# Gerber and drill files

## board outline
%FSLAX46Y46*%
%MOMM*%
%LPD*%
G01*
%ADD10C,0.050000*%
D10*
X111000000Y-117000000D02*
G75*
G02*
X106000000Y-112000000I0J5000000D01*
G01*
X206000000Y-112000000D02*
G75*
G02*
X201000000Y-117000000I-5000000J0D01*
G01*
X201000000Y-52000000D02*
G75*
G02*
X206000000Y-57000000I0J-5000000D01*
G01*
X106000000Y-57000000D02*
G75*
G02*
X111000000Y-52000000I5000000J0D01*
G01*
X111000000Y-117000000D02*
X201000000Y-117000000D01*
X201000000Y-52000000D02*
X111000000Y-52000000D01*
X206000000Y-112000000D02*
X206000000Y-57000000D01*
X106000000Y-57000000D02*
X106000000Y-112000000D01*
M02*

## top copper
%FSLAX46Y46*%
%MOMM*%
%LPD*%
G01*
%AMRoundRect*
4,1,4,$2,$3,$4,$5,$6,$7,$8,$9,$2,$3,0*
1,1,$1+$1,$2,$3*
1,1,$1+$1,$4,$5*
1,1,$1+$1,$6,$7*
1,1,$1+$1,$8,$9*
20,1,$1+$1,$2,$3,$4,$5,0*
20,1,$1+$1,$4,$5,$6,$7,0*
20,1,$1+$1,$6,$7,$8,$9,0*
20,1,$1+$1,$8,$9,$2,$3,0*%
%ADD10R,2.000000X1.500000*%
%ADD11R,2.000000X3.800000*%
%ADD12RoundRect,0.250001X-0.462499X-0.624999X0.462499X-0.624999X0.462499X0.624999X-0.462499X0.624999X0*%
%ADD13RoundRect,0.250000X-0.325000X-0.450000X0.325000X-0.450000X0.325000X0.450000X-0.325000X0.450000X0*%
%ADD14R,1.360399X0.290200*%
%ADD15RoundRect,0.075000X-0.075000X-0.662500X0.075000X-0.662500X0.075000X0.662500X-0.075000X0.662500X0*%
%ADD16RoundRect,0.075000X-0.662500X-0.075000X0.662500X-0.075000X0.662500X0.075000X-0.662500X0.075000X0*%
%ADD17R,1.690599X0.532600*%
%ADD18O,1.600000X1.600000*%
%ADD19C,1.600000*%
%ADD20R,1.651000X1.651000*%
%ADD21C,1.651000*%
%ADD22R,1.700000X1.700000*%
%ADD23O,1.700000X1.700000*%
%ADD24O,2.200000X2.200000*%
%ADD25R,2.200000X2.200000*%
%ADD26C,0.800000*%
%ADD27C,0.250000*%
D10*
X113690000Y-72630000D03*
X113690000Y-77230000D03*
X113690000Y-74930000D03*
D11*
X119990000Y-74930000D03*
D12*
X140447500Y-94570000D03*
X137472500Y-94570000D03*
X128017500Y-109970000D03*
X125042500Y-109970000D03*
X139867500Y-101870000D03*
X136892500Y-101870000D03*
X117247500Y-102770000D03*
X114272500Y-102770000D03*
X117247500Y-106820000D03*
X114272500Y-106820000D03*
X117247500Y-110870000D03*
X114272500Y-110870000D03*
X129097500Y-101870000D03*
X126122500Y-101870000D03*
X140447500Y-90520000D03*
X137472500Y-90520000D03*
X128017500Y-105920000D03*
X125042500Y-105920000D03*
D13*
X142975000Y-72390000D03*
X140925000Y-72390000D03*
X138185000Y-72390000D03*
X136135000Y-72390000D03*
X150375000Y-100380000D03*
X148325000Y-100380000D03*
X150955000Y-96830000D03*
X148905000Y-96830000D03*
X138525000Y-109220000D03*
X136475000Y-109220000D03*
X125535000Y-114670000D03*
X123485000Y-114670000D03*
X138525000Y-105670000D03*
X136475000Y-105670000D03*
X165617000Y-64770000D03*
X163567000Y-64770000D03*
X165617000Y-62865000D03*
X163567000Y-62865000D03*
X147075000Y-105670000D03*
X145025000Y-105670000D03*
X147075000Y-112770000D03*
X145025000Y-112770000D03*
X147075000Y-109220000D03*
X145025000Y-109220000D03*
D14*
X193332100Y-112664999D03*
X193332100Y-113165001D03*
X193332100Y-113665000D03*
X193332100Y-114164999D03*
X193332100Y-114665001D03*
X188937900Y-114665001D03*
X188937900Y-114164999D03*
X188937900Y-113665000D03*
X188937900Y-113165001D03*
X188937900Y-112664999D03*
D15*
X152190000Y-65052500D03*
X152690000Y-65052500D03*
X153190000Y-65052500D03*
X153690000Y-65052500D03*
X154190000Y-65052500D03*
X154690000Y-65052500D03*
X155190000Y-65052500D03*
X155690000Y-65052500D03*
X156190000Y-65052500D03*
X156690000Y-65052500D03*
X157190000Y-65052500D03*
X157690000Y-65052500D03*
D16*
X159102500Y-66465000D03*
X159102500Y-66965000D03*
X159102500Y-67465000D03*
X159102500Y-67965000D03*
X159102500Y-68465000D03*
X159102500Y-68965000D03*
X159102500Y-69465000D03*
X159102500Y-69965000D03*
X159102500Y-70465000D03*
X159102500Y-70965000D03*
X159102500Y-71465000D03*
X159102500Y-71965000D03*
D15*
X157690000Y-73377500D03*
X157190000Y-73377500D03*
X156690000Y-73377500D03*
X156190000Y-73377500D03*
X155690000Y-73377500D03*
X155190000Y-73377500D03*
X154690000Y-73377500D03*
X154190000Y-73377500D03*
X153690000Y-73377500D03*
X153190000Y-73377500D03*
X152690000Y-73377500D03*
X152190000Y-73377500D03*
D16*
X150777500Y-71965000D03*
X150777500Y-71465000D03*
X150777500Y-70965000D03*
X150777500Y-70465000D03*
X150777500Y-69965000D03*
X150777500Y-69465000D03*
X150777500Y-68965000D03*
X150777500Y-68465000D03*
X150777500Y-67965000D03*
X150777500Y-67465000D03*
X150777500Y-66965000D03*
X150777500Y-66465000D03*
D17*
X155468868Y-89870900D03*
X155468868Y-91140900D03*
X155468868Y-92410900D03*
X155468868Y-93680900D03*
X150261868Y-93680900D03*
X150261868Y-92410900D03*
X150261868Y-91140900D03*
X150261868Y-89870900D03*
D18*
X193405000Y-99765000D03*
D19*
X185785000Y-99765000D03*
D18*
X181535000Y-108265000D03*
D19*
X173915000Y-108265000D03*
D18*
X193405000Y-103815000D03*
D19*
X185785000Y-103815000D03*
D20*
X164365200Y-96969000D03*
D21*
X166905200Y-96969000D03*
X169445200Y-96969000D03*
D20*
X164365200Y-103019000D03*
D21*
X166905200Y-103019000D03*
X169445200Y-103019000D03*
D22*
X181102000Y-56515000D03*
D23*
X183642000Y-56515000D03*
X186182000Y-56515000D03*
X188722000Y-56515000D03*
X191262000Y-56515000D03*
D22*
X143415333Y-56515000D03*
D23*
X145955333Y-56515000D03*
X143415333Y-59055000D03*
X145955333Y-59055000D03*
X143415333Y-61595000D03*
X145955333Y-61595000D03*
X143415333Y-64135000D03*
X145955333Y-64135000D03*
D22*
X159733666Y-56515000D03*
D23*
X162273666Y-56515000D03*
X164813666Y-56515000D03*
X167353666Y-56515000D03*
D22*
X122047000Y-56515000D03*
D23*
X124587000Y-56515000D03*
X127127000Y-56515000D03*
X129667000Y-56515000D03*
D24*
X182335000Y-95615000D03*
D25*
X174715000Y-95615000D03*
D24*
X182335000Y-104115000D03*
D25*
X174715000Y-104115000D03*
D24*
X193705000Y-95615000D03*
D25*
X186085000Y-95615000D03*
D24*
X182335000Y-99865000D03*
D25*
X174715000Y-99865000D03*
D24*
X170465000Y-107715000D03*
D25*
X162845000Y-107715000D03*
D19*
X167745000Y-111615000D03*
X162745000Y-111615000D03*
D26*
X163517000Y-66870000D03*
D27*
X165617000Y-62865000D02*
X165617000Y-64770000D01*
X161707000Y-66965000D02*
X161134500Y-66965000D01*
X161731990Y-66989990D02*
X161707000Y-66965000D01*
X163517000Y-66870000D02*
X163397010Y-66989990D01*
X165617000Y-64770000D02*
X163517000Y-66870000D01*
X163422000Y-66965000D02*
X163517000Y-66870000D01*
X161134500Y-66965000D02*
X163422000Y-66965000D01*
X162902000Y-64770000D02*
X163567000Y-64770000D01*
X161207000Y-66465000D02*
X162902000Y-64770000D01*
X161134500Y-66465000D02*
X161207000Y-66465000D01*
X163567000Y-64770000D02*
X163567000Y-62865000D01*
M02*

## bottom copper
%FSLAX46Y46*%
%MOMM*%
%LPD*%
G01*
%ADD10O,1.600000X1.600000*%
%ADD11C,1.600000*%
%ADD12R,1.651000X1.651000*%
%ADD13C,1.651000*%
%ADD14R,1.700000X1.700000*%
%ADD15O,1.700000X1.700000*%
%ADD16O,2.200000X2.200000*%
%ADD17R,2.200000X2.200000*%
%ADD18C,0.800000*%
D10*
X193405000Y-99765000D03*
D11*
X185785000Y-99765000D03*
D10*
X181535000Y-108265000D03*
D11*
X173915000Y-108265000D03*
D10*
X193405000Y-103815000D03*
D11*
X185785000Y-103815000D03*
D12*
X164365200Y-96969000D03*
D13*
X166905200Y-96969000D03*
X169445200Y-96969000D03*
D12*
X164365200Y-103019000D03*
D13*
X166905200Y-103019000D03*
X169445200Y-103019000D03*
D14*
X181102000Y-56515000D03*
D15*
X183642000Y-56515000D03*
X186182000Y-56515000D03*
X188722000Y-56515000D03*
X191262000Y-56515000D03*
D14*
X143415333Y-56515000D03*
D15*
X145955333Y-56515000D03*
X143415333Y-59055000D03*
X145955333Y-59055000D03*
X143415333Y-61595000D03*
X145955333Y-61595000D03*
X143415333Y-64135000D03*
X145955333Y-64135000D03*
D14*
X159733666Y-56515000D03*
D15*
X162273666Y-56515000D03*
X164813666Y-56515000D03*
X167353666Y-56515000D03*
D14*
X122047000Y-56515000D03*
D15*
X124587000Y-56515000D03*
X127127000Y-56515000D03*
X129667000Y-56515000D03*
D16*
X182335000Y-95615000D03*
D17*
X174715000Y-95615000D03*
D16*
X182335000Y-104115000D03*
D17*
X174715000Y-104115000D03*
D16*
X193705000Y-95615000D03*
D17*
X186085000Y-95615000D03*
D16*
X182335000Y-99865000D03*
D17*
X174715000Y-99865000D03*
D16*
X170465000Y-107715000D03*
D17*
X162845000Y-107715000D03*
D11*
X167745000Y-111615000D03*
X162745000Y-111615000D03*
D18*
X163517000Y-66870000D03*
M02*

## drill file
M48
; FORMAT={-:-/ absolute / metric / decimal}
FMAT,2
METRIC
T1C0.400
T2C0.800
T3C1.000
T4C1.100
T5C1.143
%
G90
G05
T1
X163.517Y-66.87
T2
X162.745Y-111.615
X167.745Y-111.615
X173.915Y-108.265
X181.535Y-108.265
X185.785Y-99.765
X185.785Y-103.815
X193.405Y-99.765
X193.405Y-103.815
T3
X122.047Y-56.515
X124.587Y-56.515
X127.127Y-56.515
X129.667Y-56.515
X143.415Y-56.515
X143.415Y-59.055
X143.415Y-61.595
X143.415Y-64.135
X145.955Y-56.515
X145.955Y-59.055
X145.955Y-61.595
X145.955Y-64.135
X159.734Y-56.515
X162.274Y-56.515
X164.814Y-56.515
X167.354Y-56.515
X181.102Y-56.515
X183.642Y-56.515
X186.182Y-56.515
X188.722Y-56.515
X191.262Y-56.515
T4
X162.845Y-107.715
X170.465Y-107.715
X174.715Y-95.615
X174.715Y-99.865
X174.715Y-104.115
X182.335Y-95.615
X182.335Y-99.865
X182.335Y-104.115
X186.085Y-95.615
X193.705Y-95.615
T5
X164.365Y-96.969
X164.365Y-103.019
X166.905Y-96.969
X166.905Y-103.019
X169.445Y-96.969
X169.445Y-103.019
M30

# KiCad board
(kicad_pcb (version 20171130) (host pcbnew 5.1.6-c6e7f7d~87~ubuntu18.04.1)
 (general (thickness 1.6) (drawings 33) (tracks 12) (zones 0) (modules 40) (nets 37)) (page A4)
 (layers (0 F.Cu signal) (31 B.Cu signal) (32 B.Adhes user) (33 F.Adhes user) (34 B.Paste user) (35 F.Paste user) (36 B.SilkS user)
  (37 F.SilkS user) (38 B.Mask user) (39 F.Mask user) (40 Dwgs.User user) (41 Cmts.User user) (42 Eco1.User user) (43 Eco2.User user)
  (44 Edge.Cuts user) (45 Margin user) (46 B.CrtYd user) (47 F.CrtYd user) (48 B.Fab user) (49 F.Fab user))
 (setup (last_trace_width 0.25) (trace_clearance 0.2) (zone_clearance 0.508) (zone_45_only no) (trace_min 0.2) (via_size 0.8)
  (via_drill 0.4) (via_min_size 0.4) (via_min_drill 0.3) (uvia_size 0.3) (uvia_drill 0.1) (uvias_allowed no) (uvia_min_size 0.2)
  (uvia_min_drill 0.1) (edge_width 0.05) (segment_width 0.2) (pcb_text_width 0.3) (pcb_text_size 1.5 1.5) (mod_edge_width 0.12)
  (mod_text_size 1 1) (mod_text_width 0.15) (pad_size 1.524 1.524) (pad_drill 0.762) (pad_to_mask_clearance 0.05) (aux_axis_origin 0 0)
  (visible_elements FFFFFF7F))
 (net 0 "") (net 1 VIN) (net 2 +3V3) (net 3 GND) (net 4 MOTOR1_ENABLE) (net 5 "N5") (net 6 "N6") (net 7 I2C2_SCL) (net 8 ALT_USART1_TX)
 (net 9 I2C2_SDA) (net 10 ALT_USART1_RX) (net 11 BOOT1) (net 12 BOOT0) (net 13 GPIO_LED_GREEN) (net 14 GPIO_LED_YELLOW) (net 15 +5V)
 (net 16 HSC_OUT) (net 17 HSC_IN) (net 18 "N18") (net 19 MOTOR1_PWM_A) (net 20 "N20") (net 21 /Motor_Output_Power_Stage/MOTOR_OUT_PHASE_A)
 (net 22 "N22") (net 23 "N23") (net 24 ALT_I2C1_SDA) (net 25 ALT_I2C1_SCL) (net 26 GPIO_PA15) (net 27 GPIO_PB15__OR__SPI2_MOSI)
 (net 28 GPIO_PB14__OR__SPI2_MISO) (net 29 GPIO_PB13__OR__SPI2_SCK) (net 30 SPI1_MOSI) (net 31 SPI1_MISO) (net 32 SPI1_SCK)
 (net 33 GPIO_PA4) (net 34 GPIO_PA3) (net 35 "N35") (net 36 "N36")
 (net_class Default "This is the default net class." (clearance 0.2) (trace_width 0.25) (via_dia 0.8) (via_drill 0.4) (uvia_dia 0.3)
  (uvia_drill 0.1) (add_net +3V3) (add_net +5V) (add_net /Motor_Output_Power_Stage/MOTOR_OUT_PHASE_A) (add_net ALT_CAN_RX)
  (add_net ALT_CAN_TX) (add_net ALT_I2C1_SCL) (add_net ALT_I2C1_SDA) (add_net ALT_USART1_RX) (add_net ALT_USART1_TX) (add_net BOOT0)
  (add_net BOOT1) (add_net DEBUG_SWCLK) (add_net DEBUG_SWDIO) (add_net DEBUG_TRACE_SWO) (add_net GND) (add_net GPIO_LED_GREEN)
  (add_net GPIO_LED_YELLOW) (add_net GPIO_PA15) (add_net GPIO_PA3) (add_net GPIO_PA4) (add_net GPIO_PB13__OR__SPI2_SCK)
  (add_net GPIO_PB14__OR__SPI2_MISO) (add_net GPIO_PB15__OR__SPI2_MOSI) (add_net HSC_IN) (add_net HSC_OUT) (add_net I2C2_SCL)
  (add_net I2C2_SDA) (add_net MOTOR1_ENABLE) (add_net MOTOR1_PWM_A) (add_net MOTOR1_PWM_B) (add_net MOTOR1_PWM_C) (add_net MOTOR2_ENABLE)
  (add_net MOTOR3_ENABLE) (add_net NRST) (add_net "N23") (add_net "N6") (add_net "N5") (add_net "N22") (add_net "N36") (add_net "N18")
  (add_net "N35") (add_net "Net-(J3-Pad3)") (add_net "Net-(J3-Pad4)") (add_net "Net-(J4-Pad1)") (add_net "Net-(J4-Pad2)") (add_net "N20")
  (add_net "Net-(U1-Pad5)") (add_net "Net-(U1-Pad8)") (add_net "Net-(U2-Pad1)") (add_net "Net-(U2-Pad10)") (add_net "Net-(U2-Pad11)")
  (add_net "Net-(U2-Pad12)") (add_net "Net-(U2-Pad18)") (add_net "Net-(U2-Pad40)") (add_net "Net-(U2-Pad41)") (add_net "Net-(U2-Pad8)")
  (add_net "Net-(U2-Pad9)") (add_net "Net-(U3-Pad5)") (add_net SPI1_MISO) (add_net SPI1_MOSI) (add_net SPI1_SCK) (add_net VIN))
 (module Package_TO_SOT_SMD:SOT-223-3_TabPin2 (layer F.Cu) (at 116.84 74.93)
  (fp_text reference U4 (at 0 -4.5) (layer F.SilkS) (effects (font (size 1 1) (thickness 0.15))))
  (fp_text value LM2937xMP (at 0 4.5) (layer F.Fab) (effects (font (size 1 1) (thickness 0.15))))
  (pad 1 smd rect (at -3.15 -2.3) (size 2 1.5) (layers F.Cu F.Paste F.Mask) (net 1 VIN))
  (pad 3 smd rect (at -3.15 2.3) (size 2 1.5) (layers F.Cu F.Paste F.Mask) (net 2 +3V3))
  (pad 2 smd rect (at -3.15 0) (size 2 1.5) (layers F.Cu F.Paste F.Mask) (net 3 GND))
  (pad 2 smd rect (at 3.15 0) (size 2 3.8) (layers F.Cu F.Paste F.Mask) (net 3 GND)))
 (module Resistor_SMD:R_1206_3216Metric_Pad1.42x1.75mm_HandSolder (layer F.Cu) (at 138.96 94.57)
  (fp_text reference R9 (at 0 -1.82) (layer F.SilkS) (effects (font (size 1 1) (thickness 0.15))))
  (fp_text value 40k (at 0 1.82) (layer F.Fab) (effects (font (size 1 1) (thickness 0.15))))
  (pad 2 smd roundrect (at 1.4875 0) (size 1.425 1.75) (layers F.Cu F.Paste F.Mask) (roundrect_rratio 0.175439) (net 3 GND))
  (pad 1 smd roundrect (at -1.4875 0) (size 1.425 1.75) (layers F.Cu F.Paste F.Mask) (roundrect_rratio 0.175439) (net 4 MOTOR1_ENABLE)))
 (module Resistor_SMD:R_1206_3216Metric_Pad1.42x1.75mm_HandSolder (layer F.Cu) (at 126.53 109.97)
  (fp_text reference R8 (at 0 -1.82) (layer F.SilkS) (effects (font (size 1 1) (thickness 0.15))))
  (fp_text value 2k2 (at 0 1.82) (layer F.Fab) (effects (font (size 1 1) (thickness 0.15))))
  (pad 2 smd roundrect (at 1.4875 0) (size 1.425 1.75) (layers F.Cu F.Paste F.Mask) (roundrect_rratio 0.175439) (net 3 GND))
  (pad 1 smd roundrect (at -1.4875 0) (size 1.425 1.75) (layers F.Cu F.Paste F.Mask) (roundrect_rratio 0.175439) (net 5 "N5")))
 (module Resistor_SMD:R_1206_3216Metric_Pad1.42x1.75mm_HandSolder (layer F.Cu) (at 138.38 101.87)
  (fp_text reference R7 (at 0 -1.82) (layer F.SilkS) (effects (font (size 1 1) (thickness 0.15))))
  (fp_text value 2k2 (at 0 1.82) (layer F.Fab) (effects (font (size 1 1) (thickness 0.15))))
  (pad 2 smd roundrect (at 1.4875 0) (size 1.425 1.75) (layers F.Cu F.Paste F.Mask) (roundrect_rratio 0.175439) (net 3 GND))
  (pad 1 smd roundrect (at -1.4875 0) (size 1.425 1.75) (layers F.Cu F.Paste F.Mask) (roundrect_rratio 0.175439) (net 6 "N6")))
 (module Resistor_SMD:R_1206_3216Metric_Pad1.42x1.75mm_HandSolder (layer F.Cu) (at 115.76 102.77)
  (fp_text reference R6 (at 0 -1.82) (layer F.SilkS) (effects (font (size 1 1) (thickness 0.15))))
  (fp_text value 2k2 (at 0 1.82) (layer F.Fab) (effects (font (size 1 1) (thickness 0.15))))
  (pad 2 smd roundrect (at 1.4875 0) (size 1.425 1.75) (layers F.Cu F.Paste F.Mask) (roundrect_rratio 0.175439) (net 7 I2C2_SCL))
  (pad 1 smd roundrect (at -1.4875 0) (size 1.425 1.75) (layers F.Cu F.Paste F.Mask) (roundrect_rratio 0.175439) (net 2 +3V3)))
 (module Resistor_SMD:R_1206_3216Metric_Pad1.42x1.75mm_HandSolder (layer F.Cu) (at 115.76 106.82)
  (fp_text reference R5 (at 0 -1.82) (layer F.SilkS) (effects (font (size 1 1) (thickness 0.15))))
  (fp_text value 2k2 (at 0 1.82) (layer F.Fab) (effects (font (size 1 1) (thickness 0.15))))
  (pad 2 smd roundrect (at 1.4875 0) (size 1.425 1.75) (layers F.Cu F.Paste F.Mask) (roundrect_rratio 0.175439) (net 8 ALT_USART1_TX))
  (pad 1 smd roundrect (at -1.4875 0) (size 1.425 1.75) (layers F.Cu F.Paste F.Mask) (roundrect_rratio 0.175439) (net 2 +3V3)))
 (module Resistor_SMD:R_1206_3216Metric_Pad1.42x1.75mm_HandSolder (layer F.Cu) (at 115.76 110.87)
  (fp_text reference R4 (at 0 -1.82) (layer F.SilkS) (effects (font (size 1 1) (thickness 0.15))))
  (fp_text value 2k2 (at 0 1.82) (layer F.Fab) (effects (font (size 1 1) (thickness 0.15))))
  (pad 2 smd roundrect (at 1.4875 0) (size 1.425 1.75) (layers F.Cu F.Paste F.Mask) (roundrect_rratio 0.175439) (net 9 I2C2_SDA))
  (pad 1 smd roundrect (at -1.4875 0) (size 1.425 1.75) (layers F.Cu F.Paste F.Mask) (roundrect_rratio 0.175439) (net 2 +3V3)))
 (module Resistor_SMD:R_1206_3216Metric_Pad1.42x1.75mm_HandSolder (layer F.Cu) (at 127.61 101.87)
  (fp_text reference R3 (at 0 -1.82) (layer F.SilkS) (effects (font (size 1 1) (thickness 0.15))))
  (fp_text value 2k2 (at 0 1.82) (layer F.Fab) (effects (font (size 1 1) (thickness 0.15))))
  (pad 2 smd roundrect (at 1.4875 0) (size 1.425 1.75) (layers F.Cu F.Paste F.Mask) (roundrect_rratio 0.175439) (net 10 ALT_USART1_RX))
  (pad 1 smd roundrect (at -1.4875 0) (size 1.425 1.75) (layers F.Cu F.Paste F.Mask) (roundrect_rratio 0.175439) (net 2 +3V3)))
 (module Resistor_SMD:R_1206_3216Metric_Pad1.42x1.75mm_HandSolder (layer F.Cu) (at 138.96 90.52)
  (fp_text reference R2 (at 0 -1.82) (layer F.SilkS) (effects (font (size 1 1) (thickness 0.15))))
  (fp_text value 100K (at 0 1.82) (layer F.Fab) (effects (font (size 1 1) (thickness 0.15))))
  (pad 2 smd roundrect (at 1.4875 0) (size 1.425 1.75) (layers F.Cu F.Paste F.Mask) (roundrect_rratio 0.175439))
  (pad 1 smd roundrect (at -1.4875 0) (size 1.425 1.75) (layers F.Cu F.Paste F.Mask) (roundrect_rratio 0.175439) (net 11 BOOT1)))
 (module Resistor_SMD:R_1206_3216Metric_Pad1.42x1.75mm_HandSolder (layer F.Cu) (at 126.53 105.92)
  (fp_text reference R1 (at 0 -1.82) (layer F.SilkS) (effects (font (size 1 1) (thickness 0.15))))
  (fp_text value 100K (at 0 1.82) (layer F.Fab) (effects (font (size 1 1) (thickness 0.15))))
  (pad 2 smd roundrect (at 1.4875 0) (size 1.425 1.75) (layers F.Cu F.Paste F.Mask) (roundrect_rratio 0.175439) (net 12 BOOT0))
  (pad 1 smd roundrect (at -1.4875 0) (size 1.425 1.75) (layers F.Cu F.Paste F.Mask) (roundrect_rratio 0.175439)))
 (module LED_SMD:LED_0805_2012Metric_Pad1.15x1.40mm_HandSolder (layer F.Cu) (at 141.95 72.39)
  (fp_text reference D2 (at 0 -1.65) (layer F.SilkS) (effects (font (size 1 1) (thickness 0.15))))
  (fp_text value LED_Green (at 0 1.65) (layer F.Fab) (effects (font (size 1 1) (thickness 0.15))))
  (pad 2 smd roundrect (at 1.025 0) (size 1.15 1.4) (layers F.Cu F.Paste F.Mask) (roundrect_rratio 0.217391) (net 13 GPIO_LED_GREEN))
  (pad 1 smd roundrect (at -1.025 0) (size 1.15 1.4) (layers F.Cu F.Paste F.Mask) (roundrect_rratio 0.217391) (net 5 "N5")))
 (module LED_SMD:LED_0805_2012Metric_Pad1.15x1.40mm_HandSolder (layer F.Cu) (at 137.16 72.39)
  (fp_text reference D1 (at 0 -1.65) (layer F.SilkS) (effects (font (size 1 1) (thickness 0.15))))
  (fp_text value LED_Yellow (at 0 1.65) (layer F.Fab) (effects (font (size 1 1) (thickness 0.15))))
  (pad 2 smd roundrect (at 1.025 0) (size 1.15 1.4) (layers F.Cu F.Paste F.Mask) (roundrect_rratio 0.217391) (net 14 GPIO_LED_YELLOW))
  (pad 1 smd roundrect (at -1.025 0) (size 1.15 1.4) (layers F.Cu F.Paste F.Mask) (roundrect_rratio 0.217391) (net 6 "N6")))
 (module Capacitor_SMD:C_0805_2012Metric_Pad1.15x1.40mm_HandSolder (layer F.Cu) (at 149.35 100.38)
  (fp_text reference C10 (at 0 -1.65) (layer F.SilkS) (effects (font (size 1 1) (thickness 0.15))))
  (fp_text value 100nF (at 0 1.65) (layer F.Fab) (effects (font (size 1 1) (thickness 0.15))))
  (pad 2 smd roundrect (at 1.025 0) (size 1.15 1.4) (layers F.Cu F.Paste F.Mask) (roundrect_rratio 0.217391) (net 3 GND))
  (pad 1 smd roundrect (at -1.025 0) (size 1.15 1.4) (layers F.Cu F.Paste F.Mask) (roundrect_rratio 0.217391) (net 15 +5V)))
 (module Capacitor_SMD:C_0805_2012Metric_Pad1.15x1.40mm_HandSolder (layer F.Cu) (at 149.93 96.83)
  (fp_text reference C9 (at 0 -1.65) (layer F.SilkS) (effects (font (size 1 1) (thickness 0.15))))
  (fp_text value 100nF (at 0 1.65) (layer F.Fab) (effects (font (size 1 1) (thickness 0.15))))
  (pad 2 smd roundrect (at 1.025 0) (size 1.15 1.4) (layers F.Cu F.Paste F.Mask) (roundrect_rratio 0.217391) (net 3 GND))
  (pad 1 smd roundrect (at -1.025 0) (size 1.15 1.4) (layers F.Cu F.Paste F.Mask) (roundrect_rratio 0.217391) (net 2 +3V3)))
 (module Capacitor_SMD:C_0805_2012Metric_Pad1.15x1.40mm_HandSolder (layer F.Cu) (at 137.5 109.22)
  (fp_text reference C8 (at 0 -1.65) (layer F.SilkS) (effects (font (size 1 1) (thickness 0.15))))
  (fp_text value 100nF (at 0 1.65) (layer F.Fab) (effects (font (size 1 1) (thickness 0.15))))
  (pad 2 smd roundrect (at 1.025 0) (size 1.15 1.4) (layers F.Cu F.Paste F.Mask) (roundrect_rratio 0.217391) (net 3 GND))
  (pad 1 smd roundrect (at -1.025 0) (size 1.15 1.4) (layers F.Cu F.Paste F.Mask) (roundrect_rratio 0.217391) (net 2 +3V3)))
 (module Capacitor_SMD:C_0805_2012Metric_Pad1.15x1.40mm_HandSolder (layer F.Cu) (at 124.51 114.67)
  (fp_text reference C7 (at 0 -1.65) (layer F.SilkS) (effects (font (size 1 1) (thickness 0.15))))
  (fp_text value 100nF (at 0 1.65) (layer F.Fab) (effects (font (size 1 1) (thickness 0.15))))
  (pad 2 smd roundrect (at 1.025 0) (size 1.15 1.4) (layers F.Cu F.Paste F.Mask) (roundrect_rratio 0.217391) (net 3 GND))
  (pad 1 smd roundrect (at -1.025 0) (size 1.15 1.4) (layers F.Cu F.Paste F.Mask) (roundrect_rratio 0.217391) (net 2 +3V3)))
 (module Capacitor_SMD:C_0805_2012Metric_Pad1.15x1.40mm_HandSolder (layer F.Cu) (at 137.5 105.67)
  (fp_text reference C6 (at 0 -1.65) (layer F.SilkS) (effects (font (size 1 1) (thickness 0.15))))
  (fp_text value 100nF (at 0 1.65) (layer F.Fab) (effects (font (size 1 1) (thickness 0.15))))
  (pad 2 smd roundrect (at 1.025 0) (size 1.15 1.4) (layers F.Cu F.Paste F.Mask) (roundrect_rratio 0.217391) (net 3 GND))
  (pad 1 smd roundrect (at -1.025 0) (size 1.15 1.4) (layers F.Cu F.Paste F.Mask) (roundrect_rratio 0.217391) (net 2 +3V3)))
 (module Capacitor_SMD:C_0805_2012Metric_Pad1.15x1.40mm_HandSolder (layer F.Cu) (at 164.592 64.77)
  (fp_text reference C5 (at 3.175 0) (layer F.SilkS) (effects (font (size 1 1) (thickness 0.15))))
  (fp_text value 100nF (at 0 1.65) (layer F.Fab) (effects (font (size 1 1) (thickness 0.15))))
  (pad 2 smd roundrect (at 1.025 0) (size 1.15 1.4) (layers F.Cu F.Paste F.Mask) (roundrect_rratio 0.217391) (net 3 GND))
  (pad 1 smd roundrect (at -1.025 0) (size 1.15 1.4) (layers F.Cu F.Paste F.Mask) (roundrect_rratio 0.217391) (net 2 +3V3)))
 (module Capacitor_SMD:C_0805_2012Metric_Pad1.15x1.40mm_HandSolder (layer F.Cu) (at 164.592 62.865)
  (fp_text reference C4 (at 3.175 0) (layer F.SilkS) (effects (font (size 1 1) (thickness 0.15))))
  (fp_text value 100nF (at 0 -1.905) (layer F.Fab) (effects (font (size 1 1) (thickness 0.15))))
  (pad 2 smd roundrect (at 1.025 0) (size 1.15 1.4) (layers F.Cu F.Paste F.Mask) (roundrect_rratio 0.217391) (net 3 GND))
  (pad 1 smd roundrect (at -1.025 0) (size 1.15 1.4) (layers F.Cu F.Paste F.Mask) (roundrect_rratio 0.217391) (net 2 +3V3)))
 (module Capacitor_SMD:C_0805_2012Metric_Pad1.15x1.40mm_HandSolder (layer F.Cu) (at 146.05 105.67)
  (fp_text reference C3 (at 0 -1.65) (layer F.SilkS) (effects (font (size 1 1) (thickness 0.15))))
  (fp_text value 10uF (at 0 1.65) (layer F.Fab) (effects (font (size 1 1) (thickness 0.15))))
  (pad 2 smd roundrect (at 1.025 0) (size 1.15 1.4) (layers F.Cu F.Paste F.Mask) (roundrect_rratio 0.217391) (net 3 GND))
  (pad 1 smd roundrect (at -1.025 0) (size 1.15 1.4) (layers F.Cu F.Paste F.Mask) (roundrect_rratio 0.217391) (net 2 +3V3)))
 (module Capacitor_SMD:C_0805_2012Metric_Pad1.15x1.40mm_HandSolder (layer F.Cu) (at 146.05 112.77)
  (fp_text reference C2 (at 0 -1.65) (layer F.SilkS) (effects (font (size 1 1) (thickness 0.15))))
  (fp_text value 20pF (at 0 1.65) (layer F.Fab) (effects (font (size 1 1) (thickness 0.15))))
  (pad 2 smd roundrect (at 1.025 0) (size 1.15 1.4) (layers F.Cu F.Paste F.Mask) (roundrect_rratio 0.217391) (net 3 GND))
  (pad 1 smd roundrect (at -1.025 0) (size 1.15 1.4) (layers F.Cu F.Paste F.Mask) (roundrect_rratio 0.217391) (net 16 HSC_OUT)))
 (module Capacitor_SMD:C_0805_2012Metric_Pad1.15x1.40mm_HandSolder (layer F.Cu) (at 146.05 109.22)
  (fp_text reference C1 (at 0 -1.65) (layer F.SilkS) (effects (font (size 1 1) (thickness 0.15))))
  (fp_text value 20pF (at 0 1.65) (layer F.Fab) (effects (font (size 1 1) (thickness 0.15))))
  (pad 2 smd roundrect (at 1.025 0) (size 1.15 1.4) (layers F.Cu F.Paste F.Mask) (roundrect_rratio 0.217391) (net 3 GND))
  (pad 1 smd roundrect (at -1.025 0) (size 1.15 1.4) (layers F.Cu F.Paste F.Mask) (roundrect_rratio 0.217391) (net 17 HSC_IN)))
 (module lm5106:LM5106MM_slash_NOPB (layer F.Cu) (at 191.135 113.665)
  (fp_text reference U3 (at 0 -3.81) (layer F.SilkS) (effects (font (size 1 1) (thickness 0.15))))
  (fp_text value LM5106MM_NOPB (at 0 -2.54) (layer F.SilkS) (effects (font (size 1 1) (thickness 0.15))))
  (pad 10 smd rect (at 2.1971 -1.000001) (size 1.360399 0.2902) (layers F.Cu F.Paste F.Mask) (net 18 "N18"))
  (pad 9 smd rect (at 2.1971 -0.499999) (size 1.360399 0.2902) (layers F.Cu F.Paste F.Mask) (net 3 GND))
  (pad 8 smd rect (at 2.1971 0) (size 1.360399 0.2902) (layers F.Cu F.Paste F.Mask) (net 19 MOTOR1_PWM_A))
  (pad 7 smd rect (at 2.1971 0.499999) (size 1.360399 0.2902) (layers F.Cu F.Paste F.Mask) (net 4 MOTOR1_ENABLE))
  (pad 6 smd rect (at 2.1971 1.000001) (size 1.360399 0.2902) (layers F.Cu F.Paste F.Mask) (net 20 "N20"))
  (pad 5 smd rect (at -2.1971 1.000001) (size 1.360399 0.2902) (layers F.Cu F.Paste F.Mask))
  (pad 4 smd rect (at -2.1971 0.499999) (size 1.360399 0.2902) (layers F.Cu F.Paste F.Mask)
   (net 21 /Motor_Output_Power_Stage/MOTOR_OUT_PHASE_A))
  (pad 3 smd rect (at -2.1971 0) (size 1.360399 0.2902) (layers F.Cu F.Paste F.Mask) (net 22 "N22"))
  (pad 2 smd rect (at -2.1971 -0.499999) (size 1.360399 0.2902) (layers F.Cu F.Paste F.Mask) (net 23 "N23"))
  (pad 1 smd rect (at -2.1971 -1.000001) (size 1.360399 0.2902) (layers F.Cu F.Paste F.Mask) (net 1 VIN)))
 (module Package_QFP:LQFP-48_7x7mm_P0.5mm (layer F.Cu) (at 154.94 69.215)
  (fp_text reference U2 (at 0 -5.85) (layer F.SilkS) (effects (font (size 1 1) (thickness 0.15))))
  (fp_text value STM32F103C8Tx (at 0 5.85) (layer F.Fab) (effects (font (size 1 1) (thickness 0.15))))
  (pad 48 smd roundrect (at -2.75 -4.1625) (size 0.3 1.475) (layers F.Cu F.Paste F.Mask) (roundrect_rratio 0.25) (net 2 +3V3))
  (pad 47 smd roundrect (at -2.25 -4.1625) (size 0.3 1.475) (layers F.Cu F.Paste F.Mask) (roundrect_rratio 0.25) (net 3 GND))
  (pad 46 smd roundrect (at -1.75 -4.1625) (size 0.3 1.475) (layers F.Cu F.Paste F.Mask) (roundrect_rratio 0.25) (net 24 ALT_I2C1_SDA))
  (pad 45 smd roundrect (at -1.25 -4.1625) (size 0.3 1.475) (layers F.Cu F.Paste F.Mask) (roundrect_rratio 0.25) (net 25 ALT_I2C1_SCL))
  (pad 44 smd roundrect (at -0.75 -4.1625) (size 0.3 1.475) (layers F.Cu F.Paste F.Mask) (roundrect_rratio 0.25) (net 12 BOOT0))
  (pad 43 smd roundrect (at -0.25 -4.1625) (size 0.3 1.475) (layers F.Cu F.Paste F.Mask) (roundrect_rratio 0.25) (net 10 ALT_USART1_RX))
  (pad 42 smd roundrect (at 0.25 -4.1625) (size 0.3 1.475) (layers F.Cu F.Paste F.Mask) (roundrect_rratio 0.25) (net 8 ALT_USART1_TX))
  (pad 41 smd roundrect (at 0.75 -4.1625) (size 0.3 1.475) (layers F.Cu F.Paste F.Mask) (roundrect_rratio 0.25))
  (pad 40 smd roundrect (at 1.25 -4.1625) (size 0.3 1.475) (layers F.Cu F.Paste F.Mask) (roundrect_rratio 0.25))
  (pad 39 smd roundrect (at 1.75 -4.1625) (size 0.3 1.475) (layers F.Cu F.Paste F.Mask) (roundrect_rratio 0.25))
  (pad 38 smd roundrect (at 2.25 -4.1625) (size 0.3 1.475) (layers F.Cu F.Paste F.Mask) (roundrect_rratio 0.25) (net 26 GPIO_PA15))
  (pad 37 smd roundrect (at 2.75 -4.1625) (size 0.3 1.475) (layers F.Cu F.Paste F.Mask) (roundrect_rratio 0.25))
  (pad 36 smd roundrect (at 4.1625 -2.75) (size 1.475 0.3) (layers F.Cu F.Paste F.Mask) (roundrect_rratio 0.25) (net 2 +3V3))
  (pad 35 smd roundrect (at 4.1625 -2.25) (size 1.475 0.3) (layers F.Cu F.Paste F.Mask) (roundrect_rratio 0.25) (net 3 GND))
  (pad 34 smd roundrect (at 4.1625 -1.75) (size 1.475 0.3) (layers F.Cu F.Paste F.Mask) (roundrect_rratio 0.25))
  (pad 33 smd roundrect (at 4.1625 -1.25) (size 1.475 0.3) (layers F.Cu F.Paste F.Mask) (roundrect_rratio 0.25))
  (pad 32 smd roundrect (at 4.1625 -0.75) (size 1.475 0.3) (layers F.Cu F.Paste F.Mask) (roundrect_rratio 0.25))
  (pad 31 smd roundrect (at 4.1625 -0.25) (size 1.475 0.3) (layers F.Cu F.Paste F.Mask) (roundrect_rratio 0.25))
  (pad 30 smd roundrect (at 4.1625 0.25) (size 1.475 0.3) (layers F.Cu F.Paste F.Mask) (roundrect_rratio 0.25))
  (pad 29 smd roundrect (at 4.1625 0.75) (size 1.475 0.3) (layers F.Cu F.Paste F.Mask) (roundrect_rratio 0.25) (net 19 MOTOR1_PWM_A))
  (pad 28 smd roundrect (at 4.1625 1.25) (size 1.475 0.3) (layers F.Cu F.Paste F.Mask) (roundrect_rratio 0.25)
   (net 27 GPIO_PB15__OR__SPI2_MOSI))
  (pad 27 smd roundrect (at 4.1625 1.75) (size 1.475 0.3) (layers F.Cu F.Paste F.Mask) (roundrect_rratio 0.25)
   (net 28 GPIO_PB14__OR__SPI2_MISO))
  (pad 26 smd roundrect (at 4.1625 2.25) (size 1.475 0.3) (layers F.Cu F.Paste F.Mask) (roundrect_rratio 0.25)
   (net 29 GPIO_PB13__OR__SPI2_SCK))
  (pad 25 smd roundrect (at 4.1625 2.75) (size 1.475 0.3) (layers F.Cu F.Paste F.Mask) (roundrect_rratio 0.25) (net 4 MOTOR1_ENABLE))
  (pad 24 smd roundrect (at 2.75 4.1625) (size 0.3 1.475) (layers F.Cu F.Paste F.Mask) (roundrect_rratio 0.25) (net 2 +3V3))
  (pad 23 smd roundrect (at 2.25 4.1625) (size 0.3 1.475) (layers F.Cu F.Paste F.Mask) (roundrect_rratio 0.25) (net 3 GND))
  (pad 22 smd roundrect (at 1.75 4.1625) (size 0.3 1.475) (layers F.Cu F.Paste F.Mask) (roundrect_rratio 0.25) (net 9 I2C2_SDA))
  (pad 21 smd roundrect (at 1.25 4.1625) (size 0.3 1.475) (layers F.Cu F.Paste F.Mask) (roundrect_rratio 0.25) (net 7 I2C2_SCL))
  (pad 20 smd roundrect (at 0.75 4.1625) (size 0.3 1.475) (layers F.Cu F.Paste F.Mask) (roundrect_rratio 0.25) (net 11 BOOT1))
  (pad 19 smd roundrect (at 0.25 4.1625) (size 0.3 1.475) (layers F.Cu F.Paste F.Mask) (roundrect_rratio 0.25) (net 13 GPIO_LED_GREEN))
  (pad 18 smd roundrect (at -0.25 4.1625) (size 0.3 1.475) (layers F.Cu F.Paste F.Mask) (roundrect_rratio 0.25))
  (pad 17 smd roundrect (at -0.75 4.1625) (size 0.3 1.475) (layers F.Cu F.Paste F.Mask) (roundrect_rratio 0.25) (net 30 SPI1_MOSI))
  (pad 16 smd roundrect (at -1.25 4.1625) (size 0.3 1.475) (layers F.Cu F.Paste F.Mask) (roundrect_rratio 0.25) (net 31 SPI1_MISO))
  (pad 15 smd roundrect (at -1.75 4.1625) (size 0.3 1.475) (layers F.Cu F.Paste F.Mask) (roundrect_rratio 0.25) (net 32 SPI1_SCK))
  (pad 14 smd roundrect (at -2.25 4.1625) (size 0.3 1.475) (layers F.Cu F.Paste F.Mask) (roundrect_rratio 0.25) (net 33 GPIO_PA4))
  (pad 13 smd roundrect (at -2.75 4.1625) (size 0.3 1.475) (layers F.Cu F.Paste F.Mask) (roundrect_rratio 0.25) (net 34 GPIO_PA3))
  (pad 12 smd roundrect (at -4.1625 2.75) (size 1.475 0.3) (layers F.Cu F.Paste F.Mask) (roundrect_rratio 0.25))
  (pad 11 smd roundrect (at -4.1625 2.25) (size 1.475 0.3) (layers F.Cu F.Paste F.Mask) (roundrect_rratio 0.25))
  (pad 10 smd roundrect (at -4.1625 1.75) (size 1.475 0.3) (layers F.Cu F.Paste F.Mask) (roundrect_rratio 0.25))
  (pad 9 smd roundrect (at -4.1625 1.25) (size 1.475 0.3) (layers F.Cu F.Paste F.Mask) (roundrect_rratio 0.25))
  (pad 8 smd roundrect (at -4.1625 0.75) (size 1.475 0.3) (layers F.Cu F.Paste F.Mask) (roundrect_rratio 0.25))
  (pad 7 smd roundrect (at -4.1625 0.25) (size 1.475 0.3) (layers F.Cu F.Paste F.Mask) (roundrect_rratio 0.25))
  (pad 6 smd roundrect (at -4.1625 -0.25) (size 1.475 0.3) (layers F.Cu F.Paste F.Mask) (roundrect_rratio 0.25) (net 16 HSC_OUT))
  (pad 5 smd roundrect (at -4.1625 -0.75) (size 1.475 0.3) (layers F.Cu F.Paste F.Mask) (roundrect_rratio 0.25) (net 17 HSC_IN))
  (pad 4 smd roundrect (at -4.1625 -1.25) (size 1.475 0.3) (layers F.Cu F.Paste F.Mask) (roundrect_rratio 0.25))
  (pad 3 smd roundrect (at -4.1625 -1.75) (size 1.475 0.3) (layers F.Cu F.Paste F.Mask) (roundrect_rratio 0.25))
  (pad 2 smd roundrect (at -4.1625 -2.25) (size 1.475 0.3) (layers F.Cu F.Paste F.Mask) (roundrect_rratio 0.25) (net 14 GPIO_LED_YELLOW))
  (pad 1 smd roundrect (at -4.1625 -2.75) (size 1.475 0.3) (layers F.Cu F.Paste F.Mask) (roundrect_rratio 0.25)))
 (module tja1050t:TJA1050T (layer F.Cu) (at 152.865368 91.7759)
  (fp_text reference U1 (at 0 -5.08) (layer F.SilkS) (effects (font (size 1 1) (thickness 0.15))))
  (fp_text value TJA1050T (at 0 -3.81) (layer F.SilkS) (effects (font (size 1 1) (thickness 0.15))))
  (pad 8 smd rect (at 2.6035 -1.905) (size 1.690599 0.5326) (layers F.Cu F.Paste F.Mask))
  (pad 7 smd rect (at 2.6035 -0.635) (size 1.690599 0.5326) (layers F.Cu F.Paste F.Mask))
  (pad 6 smd rect (at 2.6035 0.635) (size 1.690599 0.5326) (layers F.Cu F.Paste F.Mask))
  (pad 5 smd rect (at 2.6035 1.905) (size 1.690599 0.5326) (layers F.Cu F.Paste F.Mask))
  (pad 4 smd rect (at -2.6035 1.905) (size 1.690599 0.5326) (layers F.Cu F.Paste F.Mask) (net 25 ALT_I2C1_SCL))
  (pad 3 smd rect (at -2.6035 0.635) (size 1.690599 0.5326) (layers F.Cu F.Paste F.Mask) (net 15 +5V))
  (pad 2 smd rect (at -2.6035 -0.635) (size 1.690599 0.5326) (layers F.Cu F.Paste F.Mask) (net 3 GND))
  (pad 1 smd rect (at -2.6035 -1.905) (size 1.690599 0.5326) (layers F.Cu F.Paste F.Mask) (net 24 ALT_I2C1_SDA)))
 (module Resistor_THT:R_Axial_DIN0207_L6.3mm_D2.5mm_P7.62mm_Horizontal (layer F.Cu) (at 185.785 99.765)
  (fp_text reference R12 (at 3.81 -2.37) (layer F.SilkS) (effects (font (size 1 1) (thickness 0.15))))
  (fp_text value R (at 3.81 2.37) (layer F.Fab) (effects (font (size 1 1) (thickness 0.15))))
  (pad 2 thru_hole oval (at 7.62 0) (size 1.6 1.6) (drill 0.8) (layers *.Cu *.Mask) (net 18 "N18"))
  (pad 1 thru_hole circle (at 0 0) (size 1.6 1.6) (drill 0.8) (layers *.Cu *.Mask) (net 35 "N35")))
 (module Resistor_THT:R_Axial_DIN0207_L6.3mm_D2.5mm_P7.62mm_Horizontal (layer F.Cu) (at 173.915 108.265)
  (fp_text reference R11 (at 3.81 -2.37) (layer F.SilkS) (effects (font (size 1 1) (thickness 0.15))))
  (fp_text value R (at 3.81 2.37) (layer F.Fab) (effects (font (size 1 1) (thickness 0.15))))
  (pad 2 thru_hole oval (at 7.62 0) (size 1.6 1.6) (drill 0.8) (layers *.Cu *.Mask) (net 22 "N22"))
  (pad 1 thru_hole circle (at 0 0) (size 1.6 1.6) (drill 0.8) (layers *.Cu *.Mask) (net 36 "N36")))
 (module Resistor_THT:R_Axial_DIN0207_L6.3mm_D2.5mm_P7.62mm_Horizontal (layer F.Cu) (at 185.785 103.815)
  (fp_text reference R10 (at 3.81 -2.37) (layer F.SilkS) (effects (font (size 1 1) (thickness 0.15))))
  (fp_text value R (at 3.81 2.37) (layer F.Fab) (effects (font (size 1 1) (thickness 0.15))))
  (pad 2 thru_hole oval (at 7.62 0) (size 1.6 1.6) (drill 0.8) (layers *.Cu *.Mask) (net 3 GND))
  (pad 1 thru_hole circle (at 0 0) (size 1.6 1.6) (drill 0.8) (layers *.Cu *.Mask) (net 20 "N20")))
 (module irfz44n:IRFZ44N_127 (layer F.Cu) (at 164.3652 96.969)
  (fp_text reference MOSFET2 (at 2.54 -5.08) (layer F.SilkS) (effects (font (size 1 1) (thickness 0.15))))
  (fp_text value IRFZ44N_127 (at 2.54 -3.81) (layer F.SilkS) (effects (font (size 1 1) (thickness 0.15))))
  (pad 1 thru_hole rect (at 0 0) (size 1.651 1.651) (drill 1.143) (layers *.Cu *.Mask) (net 35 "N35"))
  (pad 2 thru_hole circle (at 2.54 0) (size 1.651 1.651) (drill 1.143) (layers *.Cu *.Mask)
   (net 21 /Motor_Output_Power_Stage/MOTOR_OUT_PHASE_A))
  (pad 3 thru_hole circle (at 5.08 0) (size 1.651 1.651) (drill 1.143) (layers *.Cu *.Mask) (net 3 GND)))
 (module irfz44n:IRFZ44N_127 (layer F.Cu) (at 164.3652 103.019)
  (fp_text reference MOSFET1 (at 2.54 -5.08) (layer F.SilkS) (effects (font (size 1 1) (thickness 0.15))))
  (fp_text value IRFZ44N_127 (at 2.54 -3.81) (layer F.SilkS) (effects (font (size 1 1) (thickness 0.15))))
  (pad 1 thru_hole rect (at 0 0) (size 1.651 1.651) (drill 1.143) (layers *.Cu *.Mask) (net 36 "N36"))
  (pad 2 thru_hole circle (at 2.54 0) (size 1.651 1.651) (drill 1.143) (layers *.Cu *.Mask) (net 1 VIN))
  (pad 3 thru_hole circle (at 5.08 0) (size 1.651 1.651) (drill 1.143) (layers *.Cu *.Mask)
   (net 21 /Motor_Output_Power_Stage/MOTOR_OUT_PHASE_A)))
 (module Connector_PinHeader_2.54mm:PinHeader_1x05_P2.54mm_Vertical (layer F.Cu) (at 181.102 56.515 90)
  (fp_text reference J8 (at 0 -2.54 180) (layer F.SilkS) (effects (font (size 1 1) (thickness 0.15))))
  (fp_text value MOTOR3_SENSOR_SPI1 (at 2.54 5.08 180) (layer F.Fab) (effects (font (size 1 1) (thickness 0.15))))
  (pad 1 thru_hole rect (at 0 0 90) (size 1.7 1.7) (drill 1) (layers *.Cu *.Mask) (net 2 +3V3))
  (pad 2 thru_hole oval (at 0 2.54 90) (size 1.7 1.7) (drill 1) (layers *.Cu *.Mask) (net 3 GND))
  (pad 3 thru_hole oval (at 0 5.08 90) (size 1.7 1.7) (drill 1) (layers *.Cu *.Mask) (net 32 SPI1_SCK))
  (pad 4 thru_hole oval (at 0 7.62 90) (size 1.7 1.7) (drill 1) (layers *.Cu *.Mask) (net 31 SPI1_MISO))
  (pad 5 thru_hole oval (at 0 10.16 90) (size 1.7 1.7) (drill 1) (layers *.Cu *.Mask) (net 30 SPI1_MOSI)))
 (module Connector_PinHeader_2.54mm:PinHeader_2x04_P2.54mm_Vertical (layer F.Cu) (at 143.415333 56.515)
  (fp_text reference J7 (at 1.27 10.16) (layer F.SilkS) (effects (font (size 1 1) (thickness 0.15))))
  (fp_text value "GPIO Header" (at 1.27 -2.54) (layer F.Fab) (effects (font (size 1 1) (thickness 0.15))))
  (pad 1 thru_hole rect (at 0 0) (size 1.7 1.7) (drill 1) (layers *.Cu *.Mask) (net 2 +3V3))
  (pad 2 thru_hole oval (at 2.54 0) (size 1.7 1.7) (drill 1) (layers *.Cu *.Mask) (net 3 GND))
  (pad 3 thru_hole oval (at 0 2.54) (size 1.7 1.7) (drill 1) (layers *.Cu *.Mask) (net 34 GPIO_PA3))
  (pad 4 thru_hole oval (at 2.54 2.54) (size 1.7 1.7) (drill 1) (layers *.Cu *.Mask) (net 29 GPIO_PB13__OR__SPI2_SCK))
  (pad 5 thru_hole oval (at 0 5.08) (size 1.7 1.7) (drill 1) (layers *.Cu *.Mask) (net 33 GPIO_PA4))
  (pad 6 thru_hole oval (at 2.54 5.08) (size 1.7 1.7) (drill 1) (layers *.Cu *.Mask) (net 28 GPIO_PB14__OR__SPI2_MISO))
  (pad 7 thru_hole oval (at 0 7.62) (size 1.7 1.7) (drill 1) (layers *.Cu *.Mask) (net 26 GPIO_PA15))
  (pad 8 thru_hole oval (at 2.54 7.62) (size 1.7 1.7) (drill 1) (layers *.Cu *.Mask) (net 27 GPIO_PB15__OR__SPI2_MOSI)))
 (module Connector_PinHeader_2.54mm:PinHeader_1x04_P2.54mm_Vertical (layer F.Cu) (at 159.733666 56.515 90)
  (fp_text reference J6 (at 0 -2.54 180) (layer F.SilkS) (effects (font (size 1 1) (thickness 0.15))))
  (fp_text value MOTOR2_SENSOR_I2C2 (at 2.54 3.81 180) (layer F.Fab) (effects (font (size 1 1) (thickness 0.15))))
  (pad 1 thru_hole rect (at 0 0 90) (size 1.7 1.7) (drill 1) (layers *.Cu *.Mask) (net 2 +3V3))
  (pad 2 thru_hole oval (at 0 2.54 90) (size 1.7 1.7) (drill 1) (layers *.Cu *.Mask) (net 3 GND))
  (pad 3 thru_hole oval (at 0 5.08 90) (size 1.7 1.7) (drill 1) (layers *.Cu *.Mask) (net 9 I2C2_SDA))
  (pad 4 thru_hole oval (at 0 7.62 90) (size 1.7 1.7) (drill 1) (layers *.Cu *.Mask) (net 7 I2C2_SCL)))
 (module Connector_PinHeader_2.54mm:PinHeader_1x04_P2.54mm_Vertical (layer F.Cu) (at 122.047 56.515 90)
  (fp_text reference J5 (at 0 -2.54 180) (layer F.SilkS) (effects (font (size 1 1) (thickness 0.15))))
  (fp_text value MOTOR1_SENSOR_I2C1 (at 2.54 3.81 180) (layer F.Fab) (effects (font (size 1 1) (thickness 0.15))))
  (pad 1 thru_hole rect (at 0 0 90) (size 1.7 1.7) (drill 1) (layers *.Cu *.Mask) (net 2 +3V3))
  (pad 2 thru_hole oval (at 0 2.54 90) (size 1.7 1.7) (drill 1) (layers *.Cu *.Mask) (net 3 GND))
  (pad 3 thru_hole oval (at 0 5.08 90) (size 1.7 1.7) (drill 1) (layers *.Cu *.Mask) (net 10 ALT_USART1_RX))
  (pad 4 thru_hole oval (at 0 7.62 90) (size 1.7 1.7) (drill 1) (layers *.Cu *.Mask) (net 8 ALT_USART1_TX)))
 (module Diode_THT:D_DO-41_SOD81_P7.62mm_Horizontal (layer F.Cu) (at 174.715 95.615)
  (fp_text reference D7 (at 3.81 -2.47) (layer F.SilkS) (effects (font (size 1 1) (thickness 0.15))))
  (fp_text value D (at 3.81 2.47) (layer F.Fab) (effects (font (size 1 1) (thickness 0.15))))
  (pad 2 thru_hole oval (at 7.62 0) (size 2.2 2.2) (drill 1.1) (layers *.Cu *.Mask) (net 3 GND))
  (pad 1 thru_hole rect (at 0 0) (size 2.2 2.2) (drill 1.1) (layers *.Cu *.Mask) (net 21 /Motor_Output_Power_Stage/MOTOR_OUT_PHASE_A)))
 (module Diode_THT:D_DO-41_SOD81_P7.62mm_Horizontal (layer F.Cu) (at 174.715 104.115)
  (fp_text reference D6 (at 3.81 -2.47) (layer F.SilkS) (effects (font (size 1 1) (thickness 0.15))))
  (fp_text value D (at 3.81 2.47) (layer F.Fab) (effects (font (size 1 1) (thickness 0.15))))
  (pad 2 thru_hole oval (at 7.62 0) (size 2.2 2.2) (drill 1.1) (layers *.Cu *.Mask) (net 21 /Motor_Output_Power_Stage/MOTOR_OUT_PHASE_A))
  (pad 1 thru_hole rect (at 0 0) (size 2.2 2.2) (drill 1.1) (layers *.Cu *.Mask) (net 1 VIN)))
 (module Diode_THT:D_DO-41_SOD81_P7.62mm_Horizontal (layer F.Cu) (at 186.085 95.615)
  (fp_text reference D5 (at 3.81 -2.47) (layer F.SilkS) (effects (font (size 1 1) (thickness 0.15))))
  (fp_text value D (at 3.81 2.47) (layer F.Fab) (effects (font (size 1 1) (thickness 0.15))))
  (pad 2 thru_hole oval (at 7.62 0) (size 2.2 2.2) (drill 1.1) (layers *.Cu *.Mask) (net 35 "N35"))
  (pad 1 thru_hole rect (at 0 0) (size 2.2 2.2) (drill 1.1) (layers *.Cu *.Mask) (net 18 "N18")))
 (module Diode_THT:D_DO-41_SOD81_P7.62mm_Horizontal (layer F.Cu) (at 174.715 99.865)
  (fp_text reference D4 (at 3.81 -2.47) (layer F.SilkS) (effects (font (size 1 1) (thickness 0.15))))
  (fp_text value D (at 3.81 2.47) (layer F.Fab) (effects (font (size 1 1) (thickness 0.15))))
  (pad 2 thru_hole oval (at 7.62 0) (size 2.2 2.2) (drill 1.1) (layers *.Cu *.Mask) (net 36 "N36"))
  (pad 1 thru_hole rect (at 0 0) (size 2.2 2.2) (drill 1.1) (layers *.Cu *.Mask) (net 22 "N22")))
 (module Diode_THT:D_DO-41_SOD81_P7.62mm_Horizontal (layer F.Cu) (at 162.845 107.715)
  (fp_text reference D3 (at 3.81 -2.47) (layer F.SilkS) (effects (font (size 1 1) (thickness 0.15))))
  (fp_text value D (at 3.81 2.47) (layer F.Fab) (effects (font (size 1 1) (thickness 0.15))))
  (pad 2 thru_hole oval (at 7.62 0) (size 2.2 2.2) (drill 1.1) (layers *.Cu *.Mask) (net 1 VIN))
  (pad 1 thru_hole rect (at 0 0) (size 2.2 2.2) (drill 1.1) (layers *.Cu *.Mask) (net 23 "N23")))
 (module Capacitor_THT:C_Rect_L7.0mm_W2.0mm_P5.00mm (layer F.Cu) (at 162.745 111.615)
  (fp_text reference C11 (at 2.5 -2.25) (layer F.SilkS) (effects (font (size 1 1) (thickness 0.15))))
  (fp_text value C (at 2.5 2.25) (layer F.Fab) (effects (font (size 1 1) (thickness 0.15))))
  (pad 2 thru_hole circle (at 5 0) (size 1.6 1.6) (drill 0.8) (layers *.Cu *.Mask) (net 21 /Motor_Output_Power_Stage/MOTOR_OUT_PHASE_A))
  (pad 1 thru_hole circle (at 0 0) (size 1.6 1.6) (drill 0.8) (layers *.Cu *.Mask) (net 23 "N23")))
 (gr_arc (start 111 112) (end 106 112) (angle -90) (layer Edge.Cuts) (width 0.05))
 (gr_arc (start 201 112) (end 201 117) (angle -90) (layer Edge.Cuts) (width 0.05))
 (gr_arc (start 201 57) (end 206 57) (angle -90) (layer Edge.Cuts) (width 0.05))
 (gr_arc (start 111 57) (end 111 52) (angle -90) (layer Edge.Cuts) (width 0.05))
 (gr_line (start 111 117) (end 201 117) (layer Edge.Cuts) (width 0.05))
 (gr_line (start 201 52) (end 111 52) (layer Edge.Cuts) (width 0.05))
 (gr_line (start 206 112) (end 206 57) (layer Edge.Cuts) (width 0.05))
 (gr_line (start 106 57) (end 106 112) (layer Edge.Cuts) (width 0.05))
 (segment (start 165.617 62.865) (end 165.617 64.77) (width 0.25) (layer F.Cu) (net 3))
 (segment (start 161.707 66.965) (end 161.1345 66.965) (width 0.25) (layer F.Cu) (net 3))
 (segment (start 161.73199 66.98999) (end 161.707 66.965) (width 0.25) (layer F.Cu) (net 3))
 (segment (start 163.517 66.87) (end 163.39701 66.98999) (width 0.25) (layer F.Cu) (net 3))
 (via (at 163.517 66.87) (size 0.8) (drill 0.4) (layers F.Cu B.Cu) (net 3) (status 1000000))
 (segment (start 165.617 64.77) (end 163.517 66.87) (width 0.25) (layer F.Cu) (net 3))
 (segment (start 163.422 66.965) (end 163.517 66.87) (width 0.25) (layer F.Cu) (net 3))
 (segment (start 161.1345 66.965) (end 163.422 66.965) (width 0.25) (layer F.Cu) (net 3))
 (segment (start 162.902 64.77) (end 163.567 64.77) (width 0.25) (layer F.Cu) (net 2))
 (segment (start 161.207 66.465) (end 162.902 64.77) (width 0.25) (layer F.Cu) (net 2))
 (segment (start 161.1345 66.465) (end 161.207 66.465) (width 0.25) (layer F.Cu) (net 2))
 (segment (start 163.567 64.77) (end 163.567 62.865) (width 0.25) (layer F.Cu) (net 2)))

